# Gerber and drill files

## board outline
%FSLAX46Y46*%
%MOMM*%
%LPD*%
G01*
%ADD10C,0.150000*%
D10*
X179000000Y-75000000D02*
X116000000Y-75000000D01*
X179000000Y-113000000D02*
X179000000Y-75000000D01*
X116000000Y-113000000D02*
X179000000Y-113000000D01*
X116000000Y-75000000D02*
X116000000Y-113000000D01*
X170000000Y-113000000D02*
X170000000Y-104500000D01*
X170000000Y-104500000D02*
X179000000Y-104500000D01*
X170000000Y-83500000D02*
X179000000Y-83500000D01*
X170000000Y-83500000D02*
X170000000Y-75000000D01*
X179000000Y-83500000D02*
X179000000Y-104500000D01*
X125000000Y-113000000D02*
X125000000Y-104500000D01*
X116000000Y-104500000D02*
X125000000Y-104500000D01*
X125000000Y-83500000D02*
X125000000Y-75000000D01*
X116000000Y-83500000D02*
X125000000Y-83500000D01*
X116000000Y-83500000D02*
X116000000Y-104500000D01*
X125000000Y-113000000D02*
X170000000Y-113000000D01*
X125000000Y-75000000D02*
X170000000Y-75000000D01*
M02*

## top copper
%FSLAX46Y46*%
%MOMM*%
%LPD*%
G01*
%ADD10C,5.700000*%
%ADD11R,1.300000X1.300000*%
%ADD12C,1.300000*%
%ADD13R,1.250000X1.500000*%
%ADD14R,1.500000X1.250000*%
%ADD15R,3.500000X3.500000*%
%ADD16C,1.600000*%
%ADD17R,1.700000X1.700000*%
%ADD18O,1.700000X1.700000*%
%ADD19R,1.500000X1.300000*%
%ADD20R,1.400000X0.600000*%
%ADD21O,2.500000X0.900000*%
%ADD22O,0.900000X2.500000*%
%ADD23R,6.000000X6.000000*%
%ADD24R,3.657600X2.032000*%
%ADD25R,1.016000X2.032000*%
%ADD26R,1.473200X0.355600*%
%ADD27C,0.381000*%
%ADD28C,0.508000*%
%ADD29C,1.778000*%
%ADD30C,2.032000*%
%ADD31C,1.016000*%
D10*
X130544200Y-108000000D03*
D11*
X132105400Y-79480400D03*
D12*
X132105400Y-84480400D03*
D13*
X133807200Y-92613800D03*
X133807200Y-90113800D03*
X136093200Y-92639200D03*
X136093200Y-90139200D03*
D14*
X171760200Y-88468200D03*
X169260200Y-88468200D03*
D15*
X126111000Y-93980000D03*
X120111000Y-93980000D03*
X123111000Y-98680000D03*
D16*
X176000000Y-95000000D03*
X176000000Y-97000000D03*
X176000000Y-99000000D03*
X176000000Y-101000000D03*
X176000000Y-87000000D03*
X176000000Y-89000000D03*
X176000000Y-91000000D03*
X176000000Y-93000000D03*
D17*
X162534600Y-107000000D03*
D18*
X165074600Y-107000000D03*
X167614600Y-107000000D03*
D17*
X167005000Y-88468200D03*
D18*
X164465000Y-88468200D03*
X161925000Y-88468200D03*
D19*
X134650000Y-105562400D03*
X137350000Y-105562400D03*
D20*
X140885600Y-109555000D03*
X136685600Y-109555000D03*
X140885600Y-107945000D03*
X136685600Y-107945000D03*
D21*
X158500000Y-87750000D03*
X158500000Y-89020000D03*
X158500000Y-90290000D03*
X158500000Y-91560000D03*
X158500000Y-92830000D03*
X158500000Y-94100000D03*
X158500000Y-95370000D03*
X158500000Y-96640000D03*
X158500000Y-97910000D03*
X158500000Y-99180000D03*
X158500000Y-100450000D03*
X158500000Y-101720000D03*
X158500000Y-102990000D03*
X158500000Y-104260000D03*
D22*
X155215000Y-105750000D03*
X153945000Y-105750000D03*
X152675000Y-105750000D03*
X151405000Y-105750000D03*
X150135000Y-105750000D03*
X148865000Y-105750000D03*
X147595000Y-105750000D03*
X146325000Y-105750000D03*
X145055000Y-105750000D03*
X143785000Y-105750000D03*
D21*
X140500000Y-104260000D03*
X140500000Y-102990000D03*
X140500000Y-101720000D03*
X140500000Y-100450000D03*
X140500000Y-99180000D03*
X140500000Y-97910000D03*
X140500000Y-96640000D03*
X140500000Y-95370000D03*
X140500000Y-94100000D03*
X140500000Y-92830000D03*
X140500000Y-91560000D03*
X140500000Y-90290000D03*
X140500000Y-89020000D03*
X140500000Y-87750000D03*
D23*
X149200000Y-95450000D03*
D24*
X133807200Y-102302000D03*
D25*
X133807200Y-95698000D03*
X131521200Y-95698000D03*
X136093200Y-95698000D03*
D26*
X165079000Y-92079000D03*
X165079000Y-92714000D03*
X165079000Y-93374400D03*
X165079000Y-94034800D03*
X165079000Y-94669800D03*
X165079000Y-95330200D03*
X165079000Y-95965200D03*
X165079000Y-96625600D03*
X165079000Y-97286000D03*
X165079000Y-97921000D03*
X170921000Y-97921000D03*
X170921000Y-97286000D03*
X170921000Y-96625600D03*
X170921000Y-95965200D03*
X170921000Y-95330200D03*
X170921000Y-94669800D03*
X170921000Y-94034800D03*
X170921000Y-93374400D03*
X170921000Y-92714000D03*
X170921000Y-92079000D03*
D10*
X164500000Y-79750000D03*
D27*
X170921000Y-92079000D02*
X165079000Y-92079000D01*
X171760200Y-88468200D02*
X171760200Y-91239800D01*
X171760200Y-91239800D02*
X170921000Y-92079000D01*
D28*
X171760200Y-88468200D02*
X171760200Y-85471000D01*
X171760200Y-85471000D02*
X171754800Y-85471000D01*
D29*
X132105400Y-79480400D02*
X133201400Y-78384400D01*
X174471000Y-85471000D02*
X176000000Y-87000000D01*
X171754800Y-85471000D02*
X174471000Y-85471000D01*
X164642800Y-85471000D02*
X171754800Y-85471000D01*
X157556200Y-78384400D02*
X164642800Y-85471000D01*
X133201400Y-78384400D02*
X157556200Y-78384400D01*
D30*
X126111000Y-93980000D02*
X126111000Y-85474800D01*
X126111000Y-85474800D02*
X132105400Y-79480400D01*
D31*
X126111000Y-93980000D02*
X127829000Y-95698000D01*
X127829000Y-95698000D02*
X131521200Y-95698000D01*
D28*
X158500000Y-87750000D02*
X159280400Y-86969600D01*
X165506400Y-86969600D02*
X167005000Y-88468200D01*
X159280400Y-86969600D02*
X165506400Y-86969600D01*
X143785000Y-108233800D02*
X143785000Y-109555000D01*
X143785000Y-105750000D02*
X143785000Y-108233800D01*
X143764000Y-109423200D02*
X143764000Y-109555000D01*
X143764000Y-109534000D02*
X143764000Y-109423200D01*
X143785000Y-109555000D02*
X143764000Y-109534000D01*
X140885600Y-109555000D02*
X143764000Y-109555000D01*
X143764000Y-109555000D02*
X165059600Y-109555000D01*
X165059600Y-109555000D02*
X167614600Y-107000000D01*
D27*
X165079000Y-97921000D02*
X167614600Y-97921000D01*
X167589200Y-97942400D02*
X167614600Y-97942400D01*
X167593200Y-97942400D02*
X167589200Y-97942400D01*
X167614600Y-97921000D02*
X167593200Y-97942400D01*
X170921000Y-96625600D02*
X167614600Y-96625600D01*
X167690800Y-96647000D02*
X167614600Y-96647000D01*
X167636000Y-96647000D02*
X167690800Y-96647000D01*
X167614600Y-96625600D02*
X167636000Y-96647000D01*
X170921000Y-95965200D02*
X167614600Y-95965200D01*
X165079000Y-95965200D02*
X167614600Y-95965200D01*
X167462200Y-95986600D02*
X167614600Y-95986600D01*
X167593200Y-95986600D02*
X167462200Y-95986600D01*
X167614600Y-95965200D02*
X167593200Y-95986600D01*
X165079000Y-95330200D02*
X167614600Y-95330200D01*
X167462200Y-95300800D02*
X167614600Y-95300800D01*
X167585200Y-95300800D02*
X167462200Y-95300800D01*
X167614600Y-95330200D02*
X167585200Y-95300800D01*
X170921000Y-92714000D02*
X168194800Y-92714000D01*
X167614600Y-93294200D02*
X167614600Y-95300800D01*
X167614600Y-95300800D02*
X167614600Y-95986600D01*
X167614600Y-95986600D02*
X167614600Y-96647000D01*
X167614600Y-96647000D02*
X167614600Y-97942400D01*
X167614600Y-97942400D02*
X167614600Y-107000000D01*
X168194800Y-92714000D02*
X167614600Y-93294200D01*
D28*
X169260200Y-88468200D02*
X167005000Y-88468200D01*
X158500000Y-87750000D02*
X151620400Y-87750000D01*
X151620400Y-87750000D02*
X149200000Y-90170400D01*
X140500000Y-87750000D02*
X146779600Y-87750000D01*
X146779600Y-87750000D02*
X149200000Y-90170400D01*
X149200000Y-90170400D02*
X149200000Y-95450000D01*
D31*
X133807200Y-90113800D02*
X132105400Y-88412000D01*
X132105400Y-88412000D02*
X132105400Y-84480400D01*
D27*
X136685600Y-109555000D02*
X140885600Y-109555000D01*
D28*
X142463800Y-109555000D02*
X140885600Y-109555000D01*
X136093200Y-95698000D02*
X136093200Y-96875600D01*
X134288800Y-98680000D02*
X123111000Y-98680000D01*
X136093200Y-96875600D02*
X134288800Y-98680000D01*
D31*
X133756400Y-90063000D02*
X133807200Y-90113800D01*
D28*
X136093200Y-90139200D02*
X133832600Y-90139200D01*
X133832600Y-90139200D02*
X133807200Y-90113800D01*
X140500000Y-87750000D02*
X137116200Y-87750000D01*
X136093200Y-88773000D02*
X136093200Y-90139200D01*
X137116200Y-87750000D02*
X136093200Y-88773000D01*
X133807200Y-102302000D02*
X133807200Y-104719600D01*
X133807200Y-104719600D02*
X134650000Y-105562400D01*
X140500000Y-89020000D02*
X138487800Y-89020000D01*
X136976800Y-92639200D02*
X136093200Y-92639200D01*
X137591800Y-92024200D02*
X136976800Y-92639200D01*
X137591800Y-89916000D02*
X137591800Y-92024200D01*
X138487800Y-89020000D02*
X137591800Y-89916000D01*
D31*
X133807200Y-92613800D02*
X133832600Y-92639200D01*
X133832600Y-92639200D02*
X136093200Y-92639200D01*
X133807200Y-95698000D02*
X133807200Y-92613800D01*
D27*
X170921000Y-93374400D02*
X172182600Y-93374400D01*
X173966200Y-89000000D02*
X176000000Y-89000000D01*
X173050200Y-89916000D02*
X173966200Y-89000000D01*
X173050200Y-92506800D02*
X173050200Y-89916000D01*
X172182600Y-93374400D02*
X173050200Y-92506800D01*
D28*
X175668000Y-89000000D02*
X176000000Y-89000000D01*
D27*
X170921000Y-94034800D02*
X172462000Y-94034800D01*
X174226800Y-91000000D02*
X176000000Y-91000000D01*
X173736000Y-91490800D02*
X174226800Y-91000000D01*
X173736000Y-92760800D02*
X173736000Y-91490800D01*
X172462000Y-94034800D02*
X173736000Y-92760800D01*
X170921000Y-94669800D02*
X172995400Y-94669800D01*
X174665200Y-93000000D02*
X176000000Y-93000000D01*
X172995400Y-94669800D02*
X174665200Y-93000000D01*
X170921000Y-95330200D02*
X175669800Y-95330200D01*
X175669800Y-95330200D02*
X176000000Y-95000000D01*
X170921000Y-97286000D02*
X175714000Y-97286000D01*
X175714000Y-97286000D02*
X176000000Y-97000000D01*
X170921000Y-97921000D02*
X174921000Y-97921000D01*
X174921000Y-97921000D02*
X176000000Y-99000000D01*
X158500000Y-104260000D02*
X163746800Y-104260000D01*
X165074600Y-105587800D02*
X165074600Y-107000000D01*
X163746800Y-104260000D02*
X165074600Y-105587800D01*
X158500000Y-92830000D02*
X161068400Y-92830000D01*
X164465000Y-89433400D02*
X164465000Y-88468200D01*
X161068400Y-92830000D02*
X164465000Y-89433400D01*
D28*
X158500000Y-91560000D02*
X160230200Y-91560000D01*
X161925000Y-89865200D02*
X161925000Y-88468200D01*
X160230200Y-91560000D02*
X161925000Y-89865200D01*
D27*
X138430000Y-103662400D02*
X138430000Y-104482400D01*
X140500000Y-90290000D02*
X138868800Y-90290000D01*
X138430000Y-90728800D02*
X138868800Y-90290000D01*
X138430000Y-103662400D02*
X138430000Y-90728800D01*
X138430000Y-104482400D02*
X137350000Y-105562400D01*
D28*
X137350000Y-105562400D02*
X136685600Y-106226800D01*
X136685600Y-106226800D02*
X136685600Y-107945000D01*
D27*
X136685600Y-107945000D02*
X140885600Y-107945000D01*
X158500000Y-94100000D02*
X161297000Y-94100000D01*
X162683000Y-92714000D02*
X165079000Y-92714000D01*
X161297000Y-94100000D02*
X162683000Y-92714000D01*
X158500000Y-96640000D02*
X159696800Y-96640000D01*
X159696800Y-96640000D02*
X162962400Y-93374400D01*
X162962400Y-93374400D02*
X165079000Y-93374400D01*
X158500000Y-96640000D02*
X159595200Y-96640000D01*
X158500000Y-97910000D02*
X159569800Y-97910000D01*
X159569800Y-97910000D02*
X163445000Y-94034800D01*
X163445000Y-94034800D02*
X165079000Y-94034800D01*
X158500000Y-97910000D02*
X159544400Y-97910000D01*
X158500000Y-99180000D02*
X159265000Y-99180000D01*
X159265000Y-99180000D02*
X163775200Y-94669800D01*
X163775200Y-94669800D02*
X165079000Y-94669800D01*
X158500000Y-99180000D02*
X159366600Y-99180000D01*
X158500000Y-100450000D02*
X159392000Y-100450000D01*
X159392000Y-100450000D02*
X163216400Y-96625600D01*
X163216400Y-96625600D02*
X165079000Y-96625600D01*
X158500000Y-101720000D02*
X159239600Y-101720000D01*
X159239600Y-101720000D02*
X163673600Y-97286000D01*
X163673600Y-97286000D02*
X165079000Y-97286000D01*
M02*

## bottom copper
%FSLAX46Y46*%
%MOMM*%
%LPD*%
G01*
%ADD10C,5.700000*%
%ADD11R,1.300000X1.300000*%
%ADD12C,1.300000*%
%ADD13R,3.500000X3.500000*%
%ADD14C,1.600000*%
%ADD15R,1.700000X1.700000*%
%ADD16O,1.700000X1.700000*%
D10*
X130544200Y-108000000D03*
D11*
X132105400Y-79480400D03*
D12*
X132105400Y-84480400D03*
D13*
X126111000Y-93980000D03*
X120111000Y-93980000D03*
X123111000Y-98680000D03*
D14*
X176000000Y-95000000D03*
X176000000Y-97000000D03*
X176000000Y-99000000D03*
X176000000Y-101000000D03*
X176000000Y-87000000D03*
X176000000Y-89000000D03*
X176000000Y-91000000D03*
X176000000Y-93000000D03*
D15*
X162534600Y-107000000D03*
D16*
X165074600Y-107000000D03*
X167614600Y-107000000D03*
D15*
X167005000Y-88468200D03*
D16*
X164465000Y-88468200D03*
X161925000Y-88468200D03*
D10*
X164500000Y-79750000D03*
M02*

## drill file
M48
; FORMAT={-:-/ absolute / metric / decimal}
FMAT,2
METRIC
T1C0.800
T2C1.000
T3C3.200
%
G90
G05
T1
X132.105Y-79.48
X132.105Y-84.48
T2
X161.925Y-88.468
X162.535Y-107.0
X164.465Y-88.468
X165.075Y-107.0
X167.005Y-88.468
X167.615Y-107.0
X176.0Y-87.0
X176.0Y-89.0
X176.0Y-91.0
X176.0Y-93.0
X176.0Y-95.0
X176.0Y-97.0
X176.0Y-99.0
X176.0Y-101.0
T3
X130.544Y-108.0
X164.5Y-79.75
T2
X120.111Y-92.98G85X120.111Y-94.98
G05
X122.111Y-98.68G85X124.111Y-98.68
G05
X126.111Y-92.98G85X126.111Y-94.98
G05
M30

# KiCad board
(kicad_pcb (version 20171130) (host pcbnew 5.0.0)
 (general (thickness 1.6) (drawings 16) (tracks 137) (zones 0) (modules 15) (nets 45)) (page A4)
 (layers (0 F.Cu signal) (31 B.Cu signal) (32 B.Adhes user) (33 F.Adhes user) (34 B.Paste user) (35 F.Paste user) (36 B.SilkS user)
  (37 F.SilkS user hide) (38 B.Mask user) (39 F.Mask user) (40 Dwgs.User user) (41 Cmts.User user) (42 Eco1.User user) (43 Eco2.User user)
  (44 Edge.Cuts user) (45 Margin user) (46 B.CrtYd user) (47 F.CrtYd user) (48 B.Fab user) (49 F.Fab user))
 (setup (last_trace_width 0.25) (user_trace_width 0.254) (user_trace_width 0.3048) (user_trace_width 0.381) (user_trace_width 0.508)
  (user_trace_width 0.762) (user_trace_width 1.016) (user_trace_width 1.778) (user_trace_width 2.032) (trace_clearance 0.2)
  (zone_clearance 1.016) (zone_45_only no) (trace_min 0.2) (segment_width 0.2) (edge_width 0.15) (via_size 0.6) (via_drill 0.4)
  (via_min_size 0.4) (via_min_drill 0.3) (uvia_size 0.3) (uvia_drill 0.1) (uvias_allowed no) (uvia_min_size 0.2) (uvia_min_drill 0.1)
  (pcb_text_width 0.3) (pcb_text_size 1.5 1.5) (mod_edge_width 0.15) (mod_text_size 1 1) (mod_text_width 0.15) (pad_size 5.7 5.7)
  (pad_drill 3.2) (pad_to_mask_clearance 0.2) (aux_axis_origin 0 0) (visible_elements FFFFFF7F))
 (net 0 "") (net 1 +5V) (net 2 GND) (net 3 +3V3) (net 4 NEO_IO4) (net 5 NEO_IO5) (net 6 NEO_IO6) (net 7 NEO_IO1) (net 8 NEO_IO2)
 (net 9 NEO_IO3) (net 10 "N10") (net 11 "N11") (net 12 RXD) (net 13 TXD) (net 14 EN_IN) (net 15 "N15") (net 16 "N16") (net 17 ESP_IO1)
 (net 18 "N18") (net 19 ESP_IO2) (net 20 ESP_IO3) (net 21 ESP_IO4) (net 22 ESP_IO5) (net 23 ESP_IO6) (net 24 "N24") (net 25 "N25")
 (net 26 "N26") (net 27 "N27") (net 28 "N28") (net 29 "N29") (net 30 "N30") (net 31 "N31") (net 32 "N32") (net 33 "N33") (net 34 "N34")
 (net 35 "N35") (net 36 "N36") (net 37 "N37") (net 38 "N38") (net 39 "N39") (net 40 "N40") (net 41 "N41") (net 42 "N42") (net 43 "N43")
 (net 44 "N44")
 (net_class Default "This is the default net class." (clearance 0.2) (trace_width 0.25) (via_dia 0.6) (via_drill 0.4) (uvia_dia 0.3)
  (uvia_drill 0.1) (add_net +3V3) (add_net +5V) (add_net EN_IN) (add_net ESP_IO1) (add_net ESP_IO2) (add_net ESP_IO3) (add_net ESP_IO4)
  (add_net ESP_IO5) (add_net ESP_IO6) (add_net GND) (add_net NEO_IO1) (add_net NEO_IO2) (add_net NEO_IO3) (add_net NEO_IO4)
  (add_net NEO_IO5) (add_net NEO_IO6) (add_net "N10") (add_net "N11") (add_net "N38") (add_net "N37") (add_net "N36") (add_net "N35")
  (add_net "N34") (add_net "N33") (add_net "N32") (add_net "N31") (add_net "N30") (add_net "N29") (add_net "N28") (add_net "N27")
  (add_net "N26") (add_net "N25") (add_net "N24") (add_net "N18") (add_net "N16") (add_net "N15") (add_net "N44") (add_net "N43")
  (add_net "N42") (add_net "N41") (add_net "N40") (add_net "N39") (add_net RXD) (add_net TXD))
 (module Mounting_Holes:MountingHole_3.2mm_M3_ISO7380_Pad (layer F.Cu) (at 130.5 108)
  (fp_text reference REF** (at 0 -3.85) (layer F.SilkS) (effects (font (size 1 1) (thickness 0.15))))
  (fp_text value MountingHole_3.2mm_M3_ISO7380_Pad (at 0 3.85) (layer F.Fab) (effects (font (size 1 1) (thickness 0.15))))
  (pad 1 thru_hole circle (at 0.0442 0) (size 5.7 5.7) (drill 3.2) (layers *.Cu *.Mask)))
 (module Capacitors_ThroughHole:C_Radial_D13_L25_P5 (layer F.Cu) (at 132.1054 79.4804 270)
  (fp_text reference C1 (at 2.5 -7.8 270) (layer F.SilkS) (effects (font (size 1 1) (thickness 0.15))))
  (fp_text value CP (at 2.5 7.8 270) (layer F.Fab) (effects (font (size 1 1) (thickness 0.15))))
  (pad 1 thru_hole rect (at 0 0 270) (size 1.3 1.3) (drill 0.8) (layers *.Cu *.Mask) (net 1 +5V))
  (pad 2 thru_hole circle (at 5 0 270) (size 1.3 1.3) (drill 0.8) (layers *.Cu *.Mask) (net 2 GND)))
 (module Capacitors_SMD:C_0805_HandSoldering (layer F.Cu) (at 133.8072 91.3638 90)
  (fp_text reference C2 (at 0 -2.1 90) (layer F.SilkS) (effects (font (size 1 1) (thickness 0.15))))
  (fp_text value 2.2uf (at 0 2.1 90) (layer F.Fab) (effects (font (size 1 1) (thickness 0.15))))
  (pad 1 smd rect (at -1.25 0 90) (size 1.5 1.25) (layers F.Cu F.Paste F.Mask) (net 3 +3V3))
  (pad 2 smd rect (at 1.25 0 90) (size 1.5 1.25) (layers F.Cu F.Paste F.Mask) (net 2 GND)))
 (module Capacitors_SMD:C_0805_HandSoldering (layer F.Cu) (at 136.0932 91.3892 90)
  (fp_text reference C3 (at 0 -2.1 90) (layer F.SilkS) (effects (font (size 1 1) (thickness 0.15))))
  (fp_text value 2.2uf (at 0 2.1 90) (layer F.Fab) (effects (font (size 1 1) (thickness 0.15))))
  (pad 1 smd rect (at -1.25 0 90) (size 1.5 1.25) (layers F.Cu F.Paste F.Mask) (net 3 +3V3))
  (pad 2 smd rect (at 1.25 0 90) (size 1.5 1.25) (layers F.Cu F.Paste F.Mask) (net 2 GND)))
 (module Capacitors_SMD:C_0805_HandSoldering (layer F.Cu) (at 170.5102 88.4682 180)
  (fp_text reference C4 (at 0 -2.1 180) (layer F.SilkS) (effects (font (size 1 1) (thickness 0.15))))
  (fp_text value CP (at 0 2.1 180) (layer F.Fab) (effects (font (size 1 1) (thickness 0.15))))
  (pad 1 smd rect (at -1.25 0 180) (size 1.5 1.25) (layers F.Cu F.Paste F.Mask) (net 1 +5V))
  (pad 2 smd rect (at 1.25 0 180) (size 1.5 1.25) (layers F.Cu F.Paste F.Mask) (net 2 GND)))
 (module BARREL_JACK (layer F.Cu) (at 126.111 93.98)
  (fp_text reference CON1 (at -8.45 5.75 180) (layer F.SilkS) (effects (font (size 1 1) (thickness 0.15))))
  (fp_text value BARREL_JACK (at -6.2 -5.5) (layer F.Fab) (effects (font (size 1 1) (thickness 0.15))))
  (pad 1 thru_hole rect (at 0 0) (size 3.5 3.5) (drill oval 1 3) (layers *.Cu *.Mask) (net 1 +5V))
  (pad 2 thru_hole rect (at -6 0) (size 3.5 3.5) (drill oval 1 3) (layers *.Cu *.Mask) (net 2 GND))
  (pad 3 thru_hole rect (at -3 4.7) (size 3.5 3.5) (drill oval 3 1) (layers *.Cu *.Mask) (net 2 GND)))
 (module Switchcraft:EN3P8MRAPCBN (layer B.Cu) (at 176 94 270)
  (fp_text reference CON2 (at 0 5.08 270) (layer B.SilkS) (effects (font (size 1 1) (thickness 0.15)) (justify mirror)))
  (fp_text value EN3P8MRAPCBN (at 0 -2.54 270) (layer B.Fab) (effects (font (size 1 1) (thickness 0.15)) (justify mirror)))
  (pad 1 thru_hole circle (at 1 0 270) (size 1.6 1.6) (drill 1) (layers *.Cu *.Mask B.SilkS) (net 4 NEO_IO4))
  (pad 2 thru_hole circle (at 3 0 270) (size 1.6 1.6) (drill 1) (layers *.Cu *.Mask B.SilkS) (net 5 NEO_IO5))
  (pad 3 thru_hole circle (at 5 0 270) (size 1.6 1.6) (drill 1) (layers *.Cu *.Mask B.SilkS) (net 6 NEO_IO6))
  (pad 4 thru_hole circle (at 7 0 270) (size 1.6 1.6) (drill 1) (layers *.Cu *.Mask B.SilkS) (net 2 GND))
  (pad 5 thru_hole circle (at -7 0 270) (size 1.6 1.6) (drill 1) (layers *.Cu *.Mask B.SilkS) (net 1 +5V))
  (pad 6 thru_hole circle (at -5 0 270) (size 1.6 1.6) (drill 1) (layers *.Cu *.Mask B.SilkS) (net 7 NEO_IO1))
  (pad 7 thru_hole circle (at -3 0 270) (size 1.6 1.6) (drill 1) (layers *.Cu *.Mask B.SilkS) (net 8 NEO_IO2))
  (pad 8 thru_hole circle (at -1 0 270) (size 1.6 1.6) (drill 1) (layers *.Cu *.Mask B.SilkS) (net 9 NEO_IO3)))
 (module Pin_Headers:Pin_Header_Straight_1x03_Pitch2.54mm (layer F.Cu) (at 162.5346 107 90)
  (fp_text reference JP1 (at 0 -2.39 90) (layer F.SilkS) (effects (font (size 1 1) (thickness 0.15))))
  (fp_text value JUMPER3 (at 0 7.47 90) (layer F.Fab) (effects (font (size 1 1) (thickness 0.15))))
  (pad 1 thru_hole rect (at 0 0 90) (size 1.7 1.7) (drill 1) (layers *.Cu *.Mask) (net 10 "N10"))
  (pad 2 thru_hole oval (at 0 2.54 90) (size 1.7 1.7) (drill 1) (layers *.Cu *.Mask) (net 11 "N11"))
  (pad 3 thru_hole oval (at 0 5.08 90) (size 1.7 1.7) (drill 1) (layers *.Cu *.Mask) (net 2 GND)))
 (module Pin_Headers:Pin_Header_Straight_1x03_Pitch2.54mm (layer F.Cu) (at 167.005 88.4682 270)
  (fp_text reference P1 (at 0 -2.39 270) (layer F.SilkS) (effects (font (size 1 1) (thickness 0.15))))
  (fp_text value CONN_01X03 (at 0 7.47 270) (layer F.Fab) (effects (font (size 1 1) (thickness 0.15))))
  (pad 1 thru_hole rect (at 0 0 270) (size 1.7 1.7) (drill 1) (layers *.Cu *.Mask) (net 2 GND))
  (pad 2 thru_hole oval (at 0 2.54 270) (size 1.7 1.7) (drill 1) (layers *.Cu *.Mask) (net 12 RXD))
  (pad 3 thru_hole oval (at 0 5.08 270) (size 1.7 1.7) (drill 1) (layers *.Cu *.Mask) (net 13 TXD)))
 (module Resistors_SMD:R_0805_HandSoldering (layer F.Cu) (at 136 105.5624)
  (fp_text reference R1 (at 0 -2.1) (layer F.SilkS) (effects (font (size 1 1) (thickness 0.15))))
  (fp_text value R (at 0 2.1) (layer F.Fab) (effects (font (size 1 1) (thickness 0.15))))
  (pad 1 smd rect (at -1.35 0) (size 1.5 1.3) (layers F.Cu F.Paste F.Mask) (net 3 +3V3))
  (pad 2 smd rect (at 1.35 0) (size 1.5 1.3) (layers F.Cu F.Paste F.Mask) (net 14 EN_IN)))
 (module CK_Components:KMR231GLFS (layer F.Cu) (at 138.7856 108.75 180)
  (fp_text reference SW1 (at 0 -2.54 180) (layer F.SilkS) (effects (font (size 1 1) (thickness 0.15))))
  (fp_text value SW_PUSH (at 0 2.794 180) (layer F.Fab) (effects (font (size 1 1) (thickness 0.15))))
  (pad 1 smd rect (at -2.1 -0.805 180) (size 1.4 0.6) (layers F.Cu F.Paste F.Mask) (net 2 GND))
  (pad 1 smd rect (at 2.1 -0.805 180) (size 1.4 0.6) (layers F.Cu F.Paste F.Mask) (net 2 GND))
  (pad 2 smd rect (at -2.1 0.805 180) (size 1.4 0.6) (layers F.Cu F.Paste F.Mask) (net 14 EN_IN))
  (pad 2 smd rect (at 2.1 0.805 180) (size 1.4 0.6) (layers F.Cu F.Paste F.Mask) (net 14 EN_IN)))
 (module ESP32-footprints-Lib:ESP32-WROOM (layer F.Cu) (at 149.5 93 180)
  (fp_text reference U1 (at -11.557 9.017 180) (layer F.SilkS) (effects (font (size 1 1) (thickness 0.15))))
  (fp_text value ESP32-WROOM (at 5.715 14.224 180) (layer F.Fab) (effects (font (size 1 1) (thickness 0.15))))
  (pad 38 smd oval (at -9 5.25 180) (size 2.5 0.9) (layers F.Cu F.Paste F.Mask) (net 2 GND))
  (pad 37 smd oval (at -9 3.98 180) (size 2.5 0.9) (layers F.Cu F.Paste F.Mask) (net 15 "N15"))
  (pad 36 smd oval (at -9 2.71 180) (size 2.5 0.9) (layers F.Cu F.Paste F.Mask) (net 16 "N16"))
  (pad 35 smd oval (at -9 1.44 180) (size 2.5 0.9) (layers F.Cu F.Paste F.Mask) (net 13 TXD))
  (pad 34 smd oval (at -9 0.17 180) (size 2.5 0.9) (layers F.Cu F.Paste F.Mask) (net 12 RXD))
  (pad 33 smd oval (at -9 -1.1 180) (size 2.5 0.9) (layers F.Cu F.Paste F.Mask) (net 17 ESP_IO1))
  (pad 32 smd oval (at -9 -2.37 180) (size 2.5 0.9) (layers F.Cu F.Paste F.Mask) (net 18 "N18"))
  (pad 31 smd oval (at -9 -3.64 180) (size 2.5 0.9) (layers F.Cu F.Paste F.Mask) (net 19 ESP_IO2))
  (pad 30 smd oval (at -9 -4.91 180) (size 2.5 0.9) (layers F.Cu F.Paste F.Mask) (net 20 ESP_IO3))
  (pad 29 smd oval (at -9 -6.18 180) (size 2.5 0.9) (layers F.Cu F.Paste F.Mask) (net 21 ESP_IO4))
  (pad 28 smd oval (at -9 -7.45 180) (size 2.5 0.9) (layers F.Cu F.Paste F.Mask) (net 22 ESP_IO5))
  (pad 27 smd oval (at -9 -8.72 180) (size 2.5 0.9) (layers F.Cu F.Paste F.Mask) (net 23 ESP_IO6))
  (pad 26 smd oval (at -9 -9.99 180) (size 2.5 0.9) (layers F.Cu F.Paste F.Mask) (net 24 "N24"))
  (pad 25 smd oval (at -9 -11.26 180) (size 2.5 0.9) (layers F.Cu F.Paste F.Mask) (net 11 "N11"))
  (pad 24 smd oval (at -5.715 -12.75 180) (size 0.9 2.5) (layers F.Cu F.Paste F.Mask) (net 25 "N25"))
  (pad 23 smd oval (at -4.445 -12.75 180) (size 0.9 2.5) (layers F.Cu F.Paste F.Mask) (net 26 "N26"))
  (pad 22 smd oval (at -3.175 -12.75 180) (size 0.9 2.5) (layers F.Cu F.Paste F.Mask) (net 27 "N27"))
  (pad 21 smd oval (at -1.905 -12.75 180) (size 0.9 2.5) (layers F.Cu F.Paste F.Mask) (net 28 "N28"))
  (pad 20 smd oval (at -0.635 -12.75 180) (size 0.9 2.5) (layers F.Cu F.Paste F.Mask) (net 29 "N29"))
  (pad 19 smd oval (at 0.635 -12.75 180) (size 0.9 2.5) (layers F.Cu F.Paste F.Mask) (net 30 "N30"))
  (pad 18 smd oval (at 1.905 -12.75 180) (size 0.9 2.5) (layers F.Cu F.Paste F.Mask) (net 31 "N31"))
  (pad 17 smd oval (at 3.175 -12.75 180) (size 0.9 2.5) (layers F.Cu F.Paste F.Mask) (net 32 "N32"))
  (pad 16 smd oval (at 4.445 -12.75 180) (size 0.9 2.5) (layers F.Cu F.Paste F.Mask) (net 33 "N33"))
  (pad 15 smd oval (at 5.715 -12.75 180) (size 0.9 2.5) (layers F.Cu F.Paste F.Mask) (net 2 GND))
  (pad 14 smd oval (at 9 -11.26 180) (size 2.5 0.9) (layers F.Cu F.Paste F.Mask) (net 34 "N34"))
  (pad 13 smd oval (at 9 -9.99 180) (size 2.5 0.9) (layers F.Cu F.Paste F.Mask) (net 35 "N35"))
  (pad 12 smd oval (at 9 -8.72 180) (size 2.5 0.9) (layers F.Cu F.Paste F.Mask) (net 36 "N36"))
  (pad 11 smd oval (at 9 -7.45 180) (size 2.5 0.9) (layers F.Cu F.Paste F.Mask) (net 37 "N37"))
  (pad 10 smd oval (at 9 -6.18 180) (size 2.5 0.9) (layers F.Cu F.Paste F.Mask) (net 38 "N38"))
  (pad 9 smd oval (at 9 -4.91 180) (size 2.5 0.9) (layers F.Cu F.Paste F.Mask) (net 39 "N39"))
  (pad 8 smd oval (at 9 -3.64 180) (size 2.5 0.9) (layers F.Cu F.Paste F.Mask) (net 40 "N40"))
  (pad 7 smd oval (at 9 -2.37 180) (size 2.5 0.9) (layers F.Cu F.Paste F.Mask) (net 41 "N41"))
  (pad 6 smd oval (at 9 -1.1 180) (size 2.5 0.9) (layers F.Cu F.Paste F.Mask) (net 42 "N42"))
  (pad 5 smd oval (at 9 0.17 180) (size 2.5 0.9) (layers F.Cu F.Paste F.Mask) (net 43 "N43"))
  (pad 4 smd oval (at 9 1.44 180) (size 2.5 0.9) (layers F.Cu F.Paste F.Mask) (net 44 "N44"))
  (pad 3 smd oval (at 9 2.71 180) (size 2.5 0.9) (layers F.Cu F.Paste F.Mask) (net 14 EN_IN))
  (pad 2 smd oval (at 9 3.98 180) (size 2.5 0.9) (layers F.Cu F.Paste F.Mask) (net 3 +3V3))
  (pad 1 smd oval (at 9 5.25 180) (size 2.5 0.9) (layers F.Cu F.Paste F.Mask) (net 2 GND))
  (pad 39 smd rect (at 0.3 -2.45 180) (size 6 6) (layers F.Cu F.Paste F.Mask) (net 2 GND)))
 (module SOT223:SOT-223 (layer F.Cu) (at 133.8072 99 180)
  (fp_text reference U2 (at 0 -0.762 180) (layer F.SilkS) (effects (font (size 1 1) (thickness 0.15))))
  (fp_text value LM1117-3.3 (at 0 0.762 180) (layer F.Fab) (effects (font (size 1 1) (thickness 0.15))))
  (pad 2 smd rect (at 0 -3.302 180) (size 3.6576 2.032) (layers F.Cu F.Paste F.Mask) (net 3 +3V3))
  (pad 2 smd rect (at 0 3.302 180) (size 1.016 2.032) (layers F.Cu F.Paste F.Mask) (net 3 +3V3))
  (pad 3 smd rect (at 2.286 3.302 180) (size 1.016 2.032) (layers F.Cu F.Paste F.Mask) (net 1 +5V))
  (pad 1 smd rect (at -2.286 3.302 180) (size 1.016 2.032) (layers F.Cu F.Paste F.Mask) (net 2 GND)))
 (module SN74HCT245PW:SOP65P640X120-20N (layer F.Cu) (at 168 95) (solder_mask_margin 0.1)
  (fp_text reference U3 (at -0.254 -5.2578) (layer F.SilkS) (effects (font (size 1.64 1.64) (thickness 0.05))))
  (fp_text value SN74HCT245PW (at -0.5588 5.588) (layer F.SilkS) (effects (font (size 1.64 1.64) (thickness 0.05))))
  (pad 1 smd rect (at -2.921 -2.921) (size 1.4732 0.3556) (layers F.Cu F.Paste F.Mask) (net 1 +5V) (solder_mask_margin 0.2))
  (pad 2 smd rect (at -2.921 -2.286) (size 1.4732 0.3556) (layers F.Cu F.Paste F.Mask) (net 17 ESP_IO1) (solder_mask_margin 0.2))
  (pad 3 smd rect (at -2.921 -1.6256) (size 1.4732 0.3556) (layers F.Cu F.Paste F.Mask) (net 19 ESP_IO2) (solder_mask_margin 0.2))
  (pad 4 smd rect (at -2.921 -0.9652) (size 1.4732 0.3556) (layers F.Cu F.Paste F.Mask) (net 20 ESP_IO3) (solder_mask_margin 0.2))
  (pad 5 smd rect (at -2.921 -0.3302) (size 1.4732 0.3556) (layers F.Cu F.Paste F.Mask) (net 21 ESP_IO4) (solder_mask_margin 0.2))
  (pad 6 smd rect (at -2.921 0.3302) (size 1.4732 0.3556) (layers F.Cu F.Paste F.Mask) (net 2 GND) (solder_mask_margin 0.2))
  (pad 7 smd rect (at -2.921 0.9652) (size 1.4732 0.3556) (layers F.Cu F.Paste F.Mask) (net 2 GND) (solder_mask_margin 0.2))
  (pad 8 smd rect (at -2.921 1.6256) (size 1.4732 0.3556) (layers F.Cu F.Paste F.Mask) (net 22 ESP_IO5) (solder_mask_margin 0.2))
  (pad 9 smd rect (at -2.921 2.286) (size 1.4732 0.3556) (layers F.Cu F.Paste F.Mask) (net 23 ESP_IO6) (solder_mask_margin 0.2))
  (pad 10 smd rect (at -2.921 2.921) (size 1.4732 0.3556) (layers F.Cu F.Paste F.Mask) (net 2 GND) (solder_mask_margin 0.2))
  (pad 11 smd rect (at 2.921 2.921) (size 1.4732 0.3556) (layers F.Cu F.Paste F.Mask) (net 6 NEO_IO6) (solder_mask_margin 0.2))
  (pad 12 smd rect (at 2.921 2.286) (size 1.4732 0.3556) (layers F.Cu F.Paste F.Mask) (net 5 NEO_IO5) (solder_mask_margin 0.2))
  (pad 13 smd rect (at 2.921 1.6256) (size 1.4732 0.3556) (layers F.Cu F.Paste F.Mask) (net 2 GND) (solder_mask_margin 0.2))
  (pad 14 smd rect (at 2.921 0.9652) (size 1.4732 0.3556) (layers F.Cu F.Paste F.Mask) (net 2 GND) (solder_mask_margin 0.2))
  (pad 15 smd rect (at 2.921 0.3302) (size 1.4732 0.3556) (layers F.Cu F.Paste F.Mask) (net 4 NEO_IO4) (solder_mask_margin 0.2))
  (pad 16 smd rect (at 2.921 -0.3302) (size 1.4732 0.3556) (layers F.Cu F.Paste F.Mask) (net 9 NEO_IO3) (solder_mask_margin 0.2))
  (pad 17 smd rect (at 2.921 -0.9652) (size 1.4732 0.3556) (layers F.Cu F.Paste F.Mask) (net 8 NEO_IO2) (solder_mask_margin 0.2))
  (pad 18 smd rect (at 2.921 -1.6256) (size 1.4732 0.3556) (layers F.Cu F.Paste F.Mask) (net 7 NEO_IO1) (solder_mask_margin 0.2))
  (pad 19 smd rect (at 2.921 -2.286) (size 1.4732 0.3556) (layers F.Cu F.Paste F.Mask) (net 2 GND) (solder_mask_margin 0.2))
  (pad 20 smd rect (at 2.921 -2.921) (size 1.4732 0.3556) (layers F.Cu F.Paste F.Mask) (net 1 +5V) (solder_mask_margin 0.2)))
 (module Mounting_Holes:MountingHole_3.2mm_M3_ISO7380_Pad (layer F.Cu) (at 164.5 79.75)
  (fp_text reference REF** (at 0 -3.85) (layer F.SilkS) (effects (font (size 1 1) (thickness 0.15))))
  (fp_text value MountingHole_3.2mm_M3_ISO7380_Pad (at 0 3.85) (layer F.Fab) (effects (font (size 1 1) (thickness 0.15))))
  (pad 1 thru_hole circle (at 0 0) (size 5.7 5.7) (drill 3.2) (layers *.Cu *.Mask)))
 (gr_line (start 179 75) (end 116 75) (angle 90) (layer Edge.Cuts) (width 0.15))
 (gr_line (start 179 113) (end 179 75) (angle 90) (layer Edge.Cuts) (width 0.15))
 (gr_line (start 116 113) (end 179 113) (angle 90) (layer Edge.Cuts) (width 0.15))
 (gr_line (start 116 75) (end 116 113) (angle 90) (layer Edge.Cuts) (width 0.15))
 (gr_line (start 170 113) (end 170 104.5) (angle 90) (layer Edge.Cuts) (width 0.15))
 (gr_line (start 170 104.5) (end 179 104.5) (angle 90) (layer Edge.Cuts) (width 0.15))
 (gr_line (start 170 83.5) (end 179 83.5) (angle 90) (layer Edge.Cuts) (width 0.15))
 (gr_line (start 170 83.5) (end 170 75) (angle 90) (layer Edge.Cuts) (width 0.15))
 (gr_line (start 179 83.5) (end 179 104.5) (angle 90) (layer Edge.Cuts) (width 0.15))
 (gr_line (start 125 113) (end 125 104.5) (angle 90) (layer Edge.Cuts) (width 0.15))
 (gr_line (start 116 104.5) (end 125 104.5) (angle 90) (layer Edge.Cuts) (width 0.15))
 (gr_line (start 125 83.5) (end 125 75) (angle 90) (layer Edge.Cuts) (width 0.15))
 (gr_line (start 116 83.5) (end 125 83.5) (angle 90) (layer Edge.Cuts) (width 0.15))
 (gr_line (start 116 83.5) (end 116 104.5) (angle 90) (layer Edge.Cuts) (width 0.15))
 (gr_line (start 125 113) (end 170 113) (angle 90) (layer Edge.Cuts) (width 0.15))
 (gr_line (start 125 75) (end 170 75) (angle 90) (layer Edge.Cuts) (width 0.15))
 (segment (start 170.921 92.079) (end 165.079 92.079) (width 0.381) (layer F.Cu) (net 1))
 (segment (start 171.7602 88.4682) (end 171.7602 91.2398) (width 0.381) (layer F.Cu) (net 1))
 (segment (start 171.7602 91.2398) (end 170.921 92.079) (width 0.381) (layer F.Cu) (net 1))
 (segment (start 171.7602 88.4682) (end 171.7602 85.471) (width 0.508) (layer F.Cu) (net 1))
 (segment (start 171.7602 85.471) (end 171.7548 85.471) (width 0.508) (layer F.Cu) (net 1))
 (segment (start 132.1054 79.4804) (end 133.2014 78.3844) (width 1.778) (layer F.Cu) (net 1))
 (segment (start 174.471 85.471) (end 176 87) (width 1.778) (layer F.Cu) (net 1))
 (segment (start 171.7548 85.471) (end 174.471 85.471) (width 1.778) (layer F.Cu) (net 1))
 (segment (start 164.6428 85.471) (end 171.7548 85.471) (width 1.778) (layer F.Cu) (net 1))
 (segment (start 157.5562 78.3844) (end 164.6428 85.471) (width 1.778) (layer F.Cu) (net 1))
 (segment (start 133.2014 78.3844) (end 157.5562 78.3844) (width 1.778) (layer F.Cu) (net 1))
 (segment (start 126.111 93.98) (end 126.111 85.4748) (width 2.032) (layer F.Cu) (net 1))
 (segment (start 126.111 85.4748) (end 132.1054 79.4804) (width 2.032) (layer F.Cu) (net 1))
 (segment (start 126.111 93.98) (end 127.829 95.698) (width 1.016) (layer F.Cu) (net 1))
 (segment (start 127.829 95.698) (end 131.5212 95.698) (width 1.016) (layer F.Cu) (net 1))
 (segment (start 158.5 87.75) (end 159.2804 86.9696) (width 0.508) (layer F.Cu) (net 2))
 (segment (start 165.5064 86.9696) (end 167.005 88.4682) (width 0.508) (layer F.Cu) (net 2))
 (segment (start 159.2804 86.9696) (end 165.5064 86.9696) (width 0.508) (layer F.Cu) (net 2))
 (segment (start 143.785 108.2338) (end 143.785 109.555) (width 0.508) (layer F.Cu) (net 2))
 (segment (start 143.785 105.75) (end 143.785 108.2338) (width 0.508) (layer F.Cu) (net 2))
 (segment (start 143.764 109.4232) (end 143.764 109.555) (width 0.508) (layer F.Cu) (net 2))
 (segment (start 143.764 109.534) (end 143.764 109.4232) (width 0.508) (layer F.Cu) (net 2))
 (segment (start 143.785 109.555) (end 143.764 109.534) (width 0.508) (layer F.Cu) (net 2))
 (segment (start 140.8856 109.555) (end 143.764 109.555) (width 0.508) (layer F.Cu) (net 2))
 (segment (start 143.764 109.555) (end 165.0596 109.555) (width 0.508) (layer F.Cu) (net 2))
 (segment (start 165.0596 109.555) (end 167.6146 107) (width 0.508) (layer F.Cu) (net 2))
 (segment (start 165.079 97.921) (end 167.6146 97.921) (width 0.381) (layer F.Cu) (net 2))
 (segment (start 167.5892 97.9424) (end 167.6146 97.9424) (width 0.381) (layer F.Cu) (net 2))
 (segment (start 167.5932 97.9424) (end 167.5892 97.9424) (width 0.381) (layer F.Cu) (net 2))
 (segment (start 167.6146 97.921) (end 167.5932 97.9424) (width 0.381) (layer F.Cu) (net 2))
 (segment (start 170.921 96.6256) (end 167.6146 96.6256) (width 0.381) (layer F.Cu) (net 2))
 (segment (start 167.6908 96.647) (end 167.6146 96.647) (width 0.381) (layer F.Cu) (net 2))
 (segment (start 167.636 96.647) (end 167.6908 96.647) (width 0.381) (layer F.Cu) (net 2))
 (segment (start 167.6146 96.6256) (end 167.636 96.647) (width 0.381) (layer F.Cu) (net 2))
 (segment (start 170.921 95.9652) (end 167.6146 95.9652) (width 0.381) (layer F.Cu) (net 2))
 (segment (start 165.079 95.9652) (end 167.6146 95.9652) (width 0.381) (layer F.Cu) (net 2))
 (segment (start 167.4622 95.9866) (end 167.6146 95.9866) (width 0.381) (layer F.Cu) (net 2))
 (segment (start 167.5932 95.9866) (end 167.4622 95.9866) (width 0.381) (layer F.Cu) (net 2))
 (segment (start 167.6146 95.9652) (end 167.5932 95.9866) (width 0.381) (layer F.Cu) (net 2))
 (segment (start 165.079 95.3302) (end 167.6146 95.3302) (width 0.381) (layer F.Cu) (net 2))
 (segment (start 167.4622 95.3008) (end 167.6146 95.3008) (width 0.381) (layer F.Cu) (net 2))
 (segment (start 167.5852 95.3008) (end 167.4622 95.3008) (width 0.381) (layer F.Cu) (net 2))
 (segment (start 167.6146 95.3302) (end 167.5852 95.3008) (width 0.381) (layer F.Cu) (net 2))
 (segment (start 170.921 92.714) (end 168.1948 92.714) (width 0.381) (layer F.Cu) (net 2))
 (segment (start 167.6146 93.2942) (end 167.6146 95.3008) (width 0.381) (layer F.Cu) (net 2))
 (segment (start 167.6146 95.3008) (end 167.6146 95.9866) (width 0.381) (layer F.Cu) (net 2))
 (segment (start 167.6146 95.9866) (end 167.6146 96.647) (width 0.381) (layer F.Cu) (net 2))
 (segment (start 167.6146 96.647) (end 167.6146 97.9424) (width 0.381) (layer F.Cu) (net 2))
 (segment (start 167.6146 97.9424) (end 167.6146 107) (width 0.381) (layer F.Cu) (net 2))
 (segment (start 168.1948 92.714) (end 167.6146 93.2942) (width 0.381) (layer F.Cu) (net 2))
 (segment (start 169.2602 88.4682) (end 167.005 88.4682) (width 0.508) (layer F.Cu) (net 2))
 (segment (start 158.5 87.75) (end 151.6204 87.75) (width 0.508) (layer F.Cu) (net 2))
 (segment (start 151.6204 87.75) (end 149.2 90.1704) (width 0.508) (layer F.Cu) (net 2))
 (segment (start 140.5 87.75) (end 146.7796 87.75) (width 0.508) (layer F.Cu) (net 2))
 (segment (start 146.7796 87.75) (end 149.2 90.1704) (width 0.508) (layer F.Cu) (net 2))
 (segment (start 149.2 90.1704) (end 149.2 95.45) (width 0.508) (layer F.Cu) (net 2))
 (segment (start 133.8072 90.1138) (end 132.1054 88.412) (width 1.016) (layer F.Cu) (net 2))
 (segment (start 132.1054 88.412) (end 132.1054 84.4804) (width 1.016) (layer F.Cu) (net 2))
 (segment (start 136.6856 109.555) (end 140.8856 109.555) (width 0.381) (layer F.Cu) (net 2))
 (segment (start 142.4638 109.555) (end 140.8856 109.555) (width 0.508) (layer F.Cu) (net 2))
 (segment (start 136.0932 95.698) (end 136.0932 96.8756) (width 0.508) (layer F.Cu) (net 2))
 (segment (start 134.2888 98.68) (end 123.111 98.68) (width 0.508) (layer F.Cu) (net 2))
 (segment (start 136.0932 96.8756) (end 134.2888 98.68) (width 0.508) (layer F.Cu) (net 2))
 (segment (start 133.7564 90.063) (end 133.8072 90.1138) (width 1.016) (layer F.Cu) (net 2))
 (segment (start 136.0932 90.1392) (end 133.8326 90.1392) (width 0.508) (layer F.Cu) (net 2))
 (segment (start 133.8326 90.1392) (end 133.8072 90.1138) (width 0.508) (layer F.Cu) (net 2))
 (segment (start 140.5 87.75) (end 137.1162 87.75) (width 0.508) (layer F.Cu) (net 2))
 (segment (start 136.0932 88.773) (end 136.0932 90.1392) (width 0.508) (layer F.Cu) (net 2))
 (segment (start 137.1162 87.75) (end 136.0932 88.773) (width 0.508) (layer F.Cu) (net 2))
 (segment (start 133.8072 102.302) (end 133.8072 104.7196) (width 0.508) (layer F.Cu) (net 3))
 (segment (start 133.8072 104.7196) (end 134.65 105.5624) (width 0.508) (layer F.Cu) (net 3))
 (segment (start 140.5 89.02) (end 138.4878 89.02) (width 0.508) (layer F.Cu) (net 3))
 (segment (start 136.9768 92.6392) (end 136.0932 92.6392) (width 0.508) (layer F.Cu) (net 3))
 (segment (start 137.5918 92.0242) (end 136.9768 92.6392) (width 0.508) (layer F.Cu) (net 3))
 (segment (start 137.5918 89.916) (end 137.5918 92.0242) (width 0.508) (layer F.Cu) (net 3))
 (segment (start 138.4878 89.02) (end 137.5918 89.916) (width 0.508) (layer F.Cu) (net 3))
 (segment (start 133.8072 92.6138) (end 133.8326 92.6392) (width 1.016) (layer F.Cu) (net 3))
 (segment (start 133.8326 92.6392) (end 136.0932 92.6392) (width 1.016) (layer F.Cu) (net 3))
 (segment (start 133.8072 95.698) (end 133.8072 92.6138) (width 1.016) (layer F.Cu) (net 3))
 (segment (start 170.921 93.3744) (end 172.1826 93.3744) (width 0.381) (layer F.Cu) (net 7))
 (segment (start 173.9662 89) (end 176 89) (width 0.381) (layer F.Cu) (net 7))
 (segment (start 173.0502 89.916) (end 173.9662 89) (width 0.381) (layer F.Cu) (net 7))
 (segment (start 173.0502 92.5068) (end 173.0502 89.916) (width 0.381) (layer F.Cu) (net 7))
 (segment (start 172.1826 93.3744) (end 173.0502 92.5068) (width 0.381) (layer F.Cu) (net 7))
 (segment (start 175.668 89) (end 176 89) (width 0.508) (layer F.Cu) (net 7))
 (segment (start 170.921 94.0348) (end 172.462 94.0348) (width 0.381) (layer F.Cu) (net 8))
 (segment (start 174.2268 91) (end 176 91) (width 0.381) (layer F.Cu) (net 8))
 (segment (start 173.736 91.4908) (end 174.2268 91) (width 0.381) (layer F.Cu) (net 8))
 (segment (start 173.736 92.7608) (end 173.736 91.4908) (width 0.381) (layer F.Cu) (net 8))
 (segment (start 172.462 94.0348) (end 173.736 92.7608) (width 0.381) (layer F.Cu) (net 8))
 (segment (start 170.921 94.6698) (end 172.9954 94.6698) (width 0.381) (layer F.Cu) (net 9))
 (segment (start 174.6652 93) (end 176 93) (width 0.381) (layer F.Cu) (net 9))
 (segment (start 172.9954 94.6698) (end 174.6652 93) (width 0.381) (layer F.Cu) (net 9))
 (segment (start 170.921 95.3302) (end 175.6698 95.3302) (width 0.381) (layer F.Cu) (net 4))
 (segment (start 175.6698 95.3302) (end 176 95) (width 0.381) (layer F.Cu) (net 4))
 (segment (start 170.921 97.286) (end 175.714 97.286) (width 0.381) (layer F.Cu) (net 5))
 (segment (start 175.714 97.286) (end 176 97) (width 0.381) (layer F.Cu) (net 5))
 (segment (start 170.921 97.921) (end 174.921 97.921) (width 0.381) (layer F.Cu) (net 6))
 (segment (start 174.921 97.921) (end 176 99) (width 0.381) (layer F.Cu) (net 6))
 (segment (start 158.5 104.26) (end 163.7468 104.26) (width 0.381) (layer F.Cu) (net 11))
 (segment (start 165.0746 105.5878) (end 165.0746 107) (width 0.381) (layer F.Cu) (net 11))
 (segment (start 163.7468 104.26) (end 165.0746 105.5878) (width 0.381) (layer F.Cu) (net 11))
 (segment (start 158.5 92.83) (end 161.0684 92.83) (width 0.381) (layer F.Cu) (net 12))
 (segment (start 164.465 89.4334) (end 164.465 88.4682) (width 0.381) (layer F.Cu) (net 12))
 (segment (start 161.0684 92.83) (end 164.465 89.4334) (width 0.381) (layer F.Cu) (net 12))
 (segment (start 158.5 91.56) (end 160.2302 91.56) (width 0.508) (layer F.Cu) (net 13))
 (segment (start 161.925 89.8652) (end 161.925 88.4682) (width 0.508) (layer F.Cu) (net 13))
 (segment (start 160.2302 91.56) (end 161.925 89.8652) (width 0.508) (layer F.Cu) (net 13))
 (segment (start 138.43 103.6624) (end 138.43 104.4824) (width 0.381) (layer F.Cu) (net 14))
 (segment (start 140.5 90.29) (end 138.8688 90.29) (width 0.381) (layer F.Cu) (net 14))
 (segment (start 138.43 90.7288) (end 138.8688 90.29) (width 0.381) (layer F.Cu) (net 14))
 (segment (start 138.43 103.6624) (end 138.43 90.7288) (width 0.381) (layer F.Cu) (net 14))
 (segment (start 138.43 104.4824) (end 137.35 105.5624) (width 0.381) (layer F.Cu) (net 14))
 (segment (start 137.35 105.5624) (end 136.6856 106.2268) (width 0.508) (layer F.Cu) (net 14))
 (segment (start 136.6856 106.2268) (end 136.6856 107.945) (width 0.508) (layer F.Cu) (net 14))
 (segment (start 136.6856 107.945) (end 140.8856 107.945) (width 0.381) (layer F.Cu) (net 14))
 (segment (start 158.5 94.1) (end 161.297 94.1) (width 0.381) (layer F.Cu) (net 17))
 (segment (start 162.683 92.714) (end 165.079 92.714) (width 0.381) (layer F.Cu) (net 17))
 (segment (start 161.297 94.1) (end 162.683 92.714) (width 0.381) (layer F.Cu) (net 17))
 (segment (start 158.5 96.64) (end 159.6968 96.64) (width 0.381) (layer F.Cu) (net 19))
 (segment (start 159.6968 96.64) (end 162.9624 93.3744) (width 0.381) (layer F.Cu) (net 19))
 (segment (start 162.9624 93.3744) (end 165.079 93.3744) (width 0.381) (layer F.Cu) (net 19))
 (segment (start 158.5 96.64) (end 159.5952 96.64) (width 0.381) (layer F.Cu) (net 19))
 (segment (start 158.5 97.91) (end 159.5698 97.91) (width 0.381) (layer F.Cu) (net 20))
 (segment (start 159.5698 97.91) (end 163.445 94.0348) (width 0.381) (layer F.Cu) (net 20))
 (segment (start 163.445 94.0348) (end 165.079 94.0348) (width 0.381) (layer F.Cu) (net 20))
 (segment (start 158.5 97.91) (end 159.5444 97.91) (width 0.381) (layer F.Cu) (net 20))
 (segment (start 158.5 99.18) (end 159.265 99.18) (width 0.381) (layer F.Cu) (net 21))
 (segment (start 159.265 99.18) (end 163.7752 94.6698) (width 0.381) (layer F.Cu) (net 21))
 (segment (start 163.7752 94.6698) (end 165.079 94.6698) (width 0.381) (layer F.Cu) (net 21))
 (segment (start 158.5 99.18) (end 159.3666 99.18) (width 0.381) (layer F.Cu) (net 21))
 (segment (start 158.5 100.45) (end 159.392 100.45) (width 0.381) (layer F.Cu) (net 22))
 (segment (start 159.392 100.45) (end 163.2164 96.6256) (width 0.381) (layer F.Cu) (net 22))
 (segment (start 163.2164 96.6256) (end 165.079 96.6256) (width 0.381) (layer F.Cu) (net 22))
 (segment (start 158.5 101.72) (end 159.2396 101.72) (width 0.381) (layer F.Cu) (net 23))
 (segment (start 159.2396 101.72) (end 163.6736 97.286) (width 0.381) (layer F.Cu) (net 23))
 (segment (start 163.6736 97.286) (end 165.079 97.286) (width 0.381) (layer F.Cu) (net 23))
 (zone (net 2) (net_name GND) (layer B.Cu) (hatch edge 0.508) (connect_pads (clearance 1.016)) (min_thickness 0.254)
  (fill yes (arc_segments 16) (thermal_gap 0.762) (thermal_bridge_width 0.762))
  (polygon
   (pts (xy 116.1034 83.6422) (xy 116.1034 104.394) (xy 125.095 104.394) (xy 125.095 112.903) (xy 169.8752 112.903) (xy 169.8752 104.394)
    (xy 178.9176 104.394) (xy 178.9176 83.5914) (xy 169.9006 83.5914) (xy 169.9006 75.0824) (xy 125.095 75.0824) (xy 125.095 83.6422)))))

